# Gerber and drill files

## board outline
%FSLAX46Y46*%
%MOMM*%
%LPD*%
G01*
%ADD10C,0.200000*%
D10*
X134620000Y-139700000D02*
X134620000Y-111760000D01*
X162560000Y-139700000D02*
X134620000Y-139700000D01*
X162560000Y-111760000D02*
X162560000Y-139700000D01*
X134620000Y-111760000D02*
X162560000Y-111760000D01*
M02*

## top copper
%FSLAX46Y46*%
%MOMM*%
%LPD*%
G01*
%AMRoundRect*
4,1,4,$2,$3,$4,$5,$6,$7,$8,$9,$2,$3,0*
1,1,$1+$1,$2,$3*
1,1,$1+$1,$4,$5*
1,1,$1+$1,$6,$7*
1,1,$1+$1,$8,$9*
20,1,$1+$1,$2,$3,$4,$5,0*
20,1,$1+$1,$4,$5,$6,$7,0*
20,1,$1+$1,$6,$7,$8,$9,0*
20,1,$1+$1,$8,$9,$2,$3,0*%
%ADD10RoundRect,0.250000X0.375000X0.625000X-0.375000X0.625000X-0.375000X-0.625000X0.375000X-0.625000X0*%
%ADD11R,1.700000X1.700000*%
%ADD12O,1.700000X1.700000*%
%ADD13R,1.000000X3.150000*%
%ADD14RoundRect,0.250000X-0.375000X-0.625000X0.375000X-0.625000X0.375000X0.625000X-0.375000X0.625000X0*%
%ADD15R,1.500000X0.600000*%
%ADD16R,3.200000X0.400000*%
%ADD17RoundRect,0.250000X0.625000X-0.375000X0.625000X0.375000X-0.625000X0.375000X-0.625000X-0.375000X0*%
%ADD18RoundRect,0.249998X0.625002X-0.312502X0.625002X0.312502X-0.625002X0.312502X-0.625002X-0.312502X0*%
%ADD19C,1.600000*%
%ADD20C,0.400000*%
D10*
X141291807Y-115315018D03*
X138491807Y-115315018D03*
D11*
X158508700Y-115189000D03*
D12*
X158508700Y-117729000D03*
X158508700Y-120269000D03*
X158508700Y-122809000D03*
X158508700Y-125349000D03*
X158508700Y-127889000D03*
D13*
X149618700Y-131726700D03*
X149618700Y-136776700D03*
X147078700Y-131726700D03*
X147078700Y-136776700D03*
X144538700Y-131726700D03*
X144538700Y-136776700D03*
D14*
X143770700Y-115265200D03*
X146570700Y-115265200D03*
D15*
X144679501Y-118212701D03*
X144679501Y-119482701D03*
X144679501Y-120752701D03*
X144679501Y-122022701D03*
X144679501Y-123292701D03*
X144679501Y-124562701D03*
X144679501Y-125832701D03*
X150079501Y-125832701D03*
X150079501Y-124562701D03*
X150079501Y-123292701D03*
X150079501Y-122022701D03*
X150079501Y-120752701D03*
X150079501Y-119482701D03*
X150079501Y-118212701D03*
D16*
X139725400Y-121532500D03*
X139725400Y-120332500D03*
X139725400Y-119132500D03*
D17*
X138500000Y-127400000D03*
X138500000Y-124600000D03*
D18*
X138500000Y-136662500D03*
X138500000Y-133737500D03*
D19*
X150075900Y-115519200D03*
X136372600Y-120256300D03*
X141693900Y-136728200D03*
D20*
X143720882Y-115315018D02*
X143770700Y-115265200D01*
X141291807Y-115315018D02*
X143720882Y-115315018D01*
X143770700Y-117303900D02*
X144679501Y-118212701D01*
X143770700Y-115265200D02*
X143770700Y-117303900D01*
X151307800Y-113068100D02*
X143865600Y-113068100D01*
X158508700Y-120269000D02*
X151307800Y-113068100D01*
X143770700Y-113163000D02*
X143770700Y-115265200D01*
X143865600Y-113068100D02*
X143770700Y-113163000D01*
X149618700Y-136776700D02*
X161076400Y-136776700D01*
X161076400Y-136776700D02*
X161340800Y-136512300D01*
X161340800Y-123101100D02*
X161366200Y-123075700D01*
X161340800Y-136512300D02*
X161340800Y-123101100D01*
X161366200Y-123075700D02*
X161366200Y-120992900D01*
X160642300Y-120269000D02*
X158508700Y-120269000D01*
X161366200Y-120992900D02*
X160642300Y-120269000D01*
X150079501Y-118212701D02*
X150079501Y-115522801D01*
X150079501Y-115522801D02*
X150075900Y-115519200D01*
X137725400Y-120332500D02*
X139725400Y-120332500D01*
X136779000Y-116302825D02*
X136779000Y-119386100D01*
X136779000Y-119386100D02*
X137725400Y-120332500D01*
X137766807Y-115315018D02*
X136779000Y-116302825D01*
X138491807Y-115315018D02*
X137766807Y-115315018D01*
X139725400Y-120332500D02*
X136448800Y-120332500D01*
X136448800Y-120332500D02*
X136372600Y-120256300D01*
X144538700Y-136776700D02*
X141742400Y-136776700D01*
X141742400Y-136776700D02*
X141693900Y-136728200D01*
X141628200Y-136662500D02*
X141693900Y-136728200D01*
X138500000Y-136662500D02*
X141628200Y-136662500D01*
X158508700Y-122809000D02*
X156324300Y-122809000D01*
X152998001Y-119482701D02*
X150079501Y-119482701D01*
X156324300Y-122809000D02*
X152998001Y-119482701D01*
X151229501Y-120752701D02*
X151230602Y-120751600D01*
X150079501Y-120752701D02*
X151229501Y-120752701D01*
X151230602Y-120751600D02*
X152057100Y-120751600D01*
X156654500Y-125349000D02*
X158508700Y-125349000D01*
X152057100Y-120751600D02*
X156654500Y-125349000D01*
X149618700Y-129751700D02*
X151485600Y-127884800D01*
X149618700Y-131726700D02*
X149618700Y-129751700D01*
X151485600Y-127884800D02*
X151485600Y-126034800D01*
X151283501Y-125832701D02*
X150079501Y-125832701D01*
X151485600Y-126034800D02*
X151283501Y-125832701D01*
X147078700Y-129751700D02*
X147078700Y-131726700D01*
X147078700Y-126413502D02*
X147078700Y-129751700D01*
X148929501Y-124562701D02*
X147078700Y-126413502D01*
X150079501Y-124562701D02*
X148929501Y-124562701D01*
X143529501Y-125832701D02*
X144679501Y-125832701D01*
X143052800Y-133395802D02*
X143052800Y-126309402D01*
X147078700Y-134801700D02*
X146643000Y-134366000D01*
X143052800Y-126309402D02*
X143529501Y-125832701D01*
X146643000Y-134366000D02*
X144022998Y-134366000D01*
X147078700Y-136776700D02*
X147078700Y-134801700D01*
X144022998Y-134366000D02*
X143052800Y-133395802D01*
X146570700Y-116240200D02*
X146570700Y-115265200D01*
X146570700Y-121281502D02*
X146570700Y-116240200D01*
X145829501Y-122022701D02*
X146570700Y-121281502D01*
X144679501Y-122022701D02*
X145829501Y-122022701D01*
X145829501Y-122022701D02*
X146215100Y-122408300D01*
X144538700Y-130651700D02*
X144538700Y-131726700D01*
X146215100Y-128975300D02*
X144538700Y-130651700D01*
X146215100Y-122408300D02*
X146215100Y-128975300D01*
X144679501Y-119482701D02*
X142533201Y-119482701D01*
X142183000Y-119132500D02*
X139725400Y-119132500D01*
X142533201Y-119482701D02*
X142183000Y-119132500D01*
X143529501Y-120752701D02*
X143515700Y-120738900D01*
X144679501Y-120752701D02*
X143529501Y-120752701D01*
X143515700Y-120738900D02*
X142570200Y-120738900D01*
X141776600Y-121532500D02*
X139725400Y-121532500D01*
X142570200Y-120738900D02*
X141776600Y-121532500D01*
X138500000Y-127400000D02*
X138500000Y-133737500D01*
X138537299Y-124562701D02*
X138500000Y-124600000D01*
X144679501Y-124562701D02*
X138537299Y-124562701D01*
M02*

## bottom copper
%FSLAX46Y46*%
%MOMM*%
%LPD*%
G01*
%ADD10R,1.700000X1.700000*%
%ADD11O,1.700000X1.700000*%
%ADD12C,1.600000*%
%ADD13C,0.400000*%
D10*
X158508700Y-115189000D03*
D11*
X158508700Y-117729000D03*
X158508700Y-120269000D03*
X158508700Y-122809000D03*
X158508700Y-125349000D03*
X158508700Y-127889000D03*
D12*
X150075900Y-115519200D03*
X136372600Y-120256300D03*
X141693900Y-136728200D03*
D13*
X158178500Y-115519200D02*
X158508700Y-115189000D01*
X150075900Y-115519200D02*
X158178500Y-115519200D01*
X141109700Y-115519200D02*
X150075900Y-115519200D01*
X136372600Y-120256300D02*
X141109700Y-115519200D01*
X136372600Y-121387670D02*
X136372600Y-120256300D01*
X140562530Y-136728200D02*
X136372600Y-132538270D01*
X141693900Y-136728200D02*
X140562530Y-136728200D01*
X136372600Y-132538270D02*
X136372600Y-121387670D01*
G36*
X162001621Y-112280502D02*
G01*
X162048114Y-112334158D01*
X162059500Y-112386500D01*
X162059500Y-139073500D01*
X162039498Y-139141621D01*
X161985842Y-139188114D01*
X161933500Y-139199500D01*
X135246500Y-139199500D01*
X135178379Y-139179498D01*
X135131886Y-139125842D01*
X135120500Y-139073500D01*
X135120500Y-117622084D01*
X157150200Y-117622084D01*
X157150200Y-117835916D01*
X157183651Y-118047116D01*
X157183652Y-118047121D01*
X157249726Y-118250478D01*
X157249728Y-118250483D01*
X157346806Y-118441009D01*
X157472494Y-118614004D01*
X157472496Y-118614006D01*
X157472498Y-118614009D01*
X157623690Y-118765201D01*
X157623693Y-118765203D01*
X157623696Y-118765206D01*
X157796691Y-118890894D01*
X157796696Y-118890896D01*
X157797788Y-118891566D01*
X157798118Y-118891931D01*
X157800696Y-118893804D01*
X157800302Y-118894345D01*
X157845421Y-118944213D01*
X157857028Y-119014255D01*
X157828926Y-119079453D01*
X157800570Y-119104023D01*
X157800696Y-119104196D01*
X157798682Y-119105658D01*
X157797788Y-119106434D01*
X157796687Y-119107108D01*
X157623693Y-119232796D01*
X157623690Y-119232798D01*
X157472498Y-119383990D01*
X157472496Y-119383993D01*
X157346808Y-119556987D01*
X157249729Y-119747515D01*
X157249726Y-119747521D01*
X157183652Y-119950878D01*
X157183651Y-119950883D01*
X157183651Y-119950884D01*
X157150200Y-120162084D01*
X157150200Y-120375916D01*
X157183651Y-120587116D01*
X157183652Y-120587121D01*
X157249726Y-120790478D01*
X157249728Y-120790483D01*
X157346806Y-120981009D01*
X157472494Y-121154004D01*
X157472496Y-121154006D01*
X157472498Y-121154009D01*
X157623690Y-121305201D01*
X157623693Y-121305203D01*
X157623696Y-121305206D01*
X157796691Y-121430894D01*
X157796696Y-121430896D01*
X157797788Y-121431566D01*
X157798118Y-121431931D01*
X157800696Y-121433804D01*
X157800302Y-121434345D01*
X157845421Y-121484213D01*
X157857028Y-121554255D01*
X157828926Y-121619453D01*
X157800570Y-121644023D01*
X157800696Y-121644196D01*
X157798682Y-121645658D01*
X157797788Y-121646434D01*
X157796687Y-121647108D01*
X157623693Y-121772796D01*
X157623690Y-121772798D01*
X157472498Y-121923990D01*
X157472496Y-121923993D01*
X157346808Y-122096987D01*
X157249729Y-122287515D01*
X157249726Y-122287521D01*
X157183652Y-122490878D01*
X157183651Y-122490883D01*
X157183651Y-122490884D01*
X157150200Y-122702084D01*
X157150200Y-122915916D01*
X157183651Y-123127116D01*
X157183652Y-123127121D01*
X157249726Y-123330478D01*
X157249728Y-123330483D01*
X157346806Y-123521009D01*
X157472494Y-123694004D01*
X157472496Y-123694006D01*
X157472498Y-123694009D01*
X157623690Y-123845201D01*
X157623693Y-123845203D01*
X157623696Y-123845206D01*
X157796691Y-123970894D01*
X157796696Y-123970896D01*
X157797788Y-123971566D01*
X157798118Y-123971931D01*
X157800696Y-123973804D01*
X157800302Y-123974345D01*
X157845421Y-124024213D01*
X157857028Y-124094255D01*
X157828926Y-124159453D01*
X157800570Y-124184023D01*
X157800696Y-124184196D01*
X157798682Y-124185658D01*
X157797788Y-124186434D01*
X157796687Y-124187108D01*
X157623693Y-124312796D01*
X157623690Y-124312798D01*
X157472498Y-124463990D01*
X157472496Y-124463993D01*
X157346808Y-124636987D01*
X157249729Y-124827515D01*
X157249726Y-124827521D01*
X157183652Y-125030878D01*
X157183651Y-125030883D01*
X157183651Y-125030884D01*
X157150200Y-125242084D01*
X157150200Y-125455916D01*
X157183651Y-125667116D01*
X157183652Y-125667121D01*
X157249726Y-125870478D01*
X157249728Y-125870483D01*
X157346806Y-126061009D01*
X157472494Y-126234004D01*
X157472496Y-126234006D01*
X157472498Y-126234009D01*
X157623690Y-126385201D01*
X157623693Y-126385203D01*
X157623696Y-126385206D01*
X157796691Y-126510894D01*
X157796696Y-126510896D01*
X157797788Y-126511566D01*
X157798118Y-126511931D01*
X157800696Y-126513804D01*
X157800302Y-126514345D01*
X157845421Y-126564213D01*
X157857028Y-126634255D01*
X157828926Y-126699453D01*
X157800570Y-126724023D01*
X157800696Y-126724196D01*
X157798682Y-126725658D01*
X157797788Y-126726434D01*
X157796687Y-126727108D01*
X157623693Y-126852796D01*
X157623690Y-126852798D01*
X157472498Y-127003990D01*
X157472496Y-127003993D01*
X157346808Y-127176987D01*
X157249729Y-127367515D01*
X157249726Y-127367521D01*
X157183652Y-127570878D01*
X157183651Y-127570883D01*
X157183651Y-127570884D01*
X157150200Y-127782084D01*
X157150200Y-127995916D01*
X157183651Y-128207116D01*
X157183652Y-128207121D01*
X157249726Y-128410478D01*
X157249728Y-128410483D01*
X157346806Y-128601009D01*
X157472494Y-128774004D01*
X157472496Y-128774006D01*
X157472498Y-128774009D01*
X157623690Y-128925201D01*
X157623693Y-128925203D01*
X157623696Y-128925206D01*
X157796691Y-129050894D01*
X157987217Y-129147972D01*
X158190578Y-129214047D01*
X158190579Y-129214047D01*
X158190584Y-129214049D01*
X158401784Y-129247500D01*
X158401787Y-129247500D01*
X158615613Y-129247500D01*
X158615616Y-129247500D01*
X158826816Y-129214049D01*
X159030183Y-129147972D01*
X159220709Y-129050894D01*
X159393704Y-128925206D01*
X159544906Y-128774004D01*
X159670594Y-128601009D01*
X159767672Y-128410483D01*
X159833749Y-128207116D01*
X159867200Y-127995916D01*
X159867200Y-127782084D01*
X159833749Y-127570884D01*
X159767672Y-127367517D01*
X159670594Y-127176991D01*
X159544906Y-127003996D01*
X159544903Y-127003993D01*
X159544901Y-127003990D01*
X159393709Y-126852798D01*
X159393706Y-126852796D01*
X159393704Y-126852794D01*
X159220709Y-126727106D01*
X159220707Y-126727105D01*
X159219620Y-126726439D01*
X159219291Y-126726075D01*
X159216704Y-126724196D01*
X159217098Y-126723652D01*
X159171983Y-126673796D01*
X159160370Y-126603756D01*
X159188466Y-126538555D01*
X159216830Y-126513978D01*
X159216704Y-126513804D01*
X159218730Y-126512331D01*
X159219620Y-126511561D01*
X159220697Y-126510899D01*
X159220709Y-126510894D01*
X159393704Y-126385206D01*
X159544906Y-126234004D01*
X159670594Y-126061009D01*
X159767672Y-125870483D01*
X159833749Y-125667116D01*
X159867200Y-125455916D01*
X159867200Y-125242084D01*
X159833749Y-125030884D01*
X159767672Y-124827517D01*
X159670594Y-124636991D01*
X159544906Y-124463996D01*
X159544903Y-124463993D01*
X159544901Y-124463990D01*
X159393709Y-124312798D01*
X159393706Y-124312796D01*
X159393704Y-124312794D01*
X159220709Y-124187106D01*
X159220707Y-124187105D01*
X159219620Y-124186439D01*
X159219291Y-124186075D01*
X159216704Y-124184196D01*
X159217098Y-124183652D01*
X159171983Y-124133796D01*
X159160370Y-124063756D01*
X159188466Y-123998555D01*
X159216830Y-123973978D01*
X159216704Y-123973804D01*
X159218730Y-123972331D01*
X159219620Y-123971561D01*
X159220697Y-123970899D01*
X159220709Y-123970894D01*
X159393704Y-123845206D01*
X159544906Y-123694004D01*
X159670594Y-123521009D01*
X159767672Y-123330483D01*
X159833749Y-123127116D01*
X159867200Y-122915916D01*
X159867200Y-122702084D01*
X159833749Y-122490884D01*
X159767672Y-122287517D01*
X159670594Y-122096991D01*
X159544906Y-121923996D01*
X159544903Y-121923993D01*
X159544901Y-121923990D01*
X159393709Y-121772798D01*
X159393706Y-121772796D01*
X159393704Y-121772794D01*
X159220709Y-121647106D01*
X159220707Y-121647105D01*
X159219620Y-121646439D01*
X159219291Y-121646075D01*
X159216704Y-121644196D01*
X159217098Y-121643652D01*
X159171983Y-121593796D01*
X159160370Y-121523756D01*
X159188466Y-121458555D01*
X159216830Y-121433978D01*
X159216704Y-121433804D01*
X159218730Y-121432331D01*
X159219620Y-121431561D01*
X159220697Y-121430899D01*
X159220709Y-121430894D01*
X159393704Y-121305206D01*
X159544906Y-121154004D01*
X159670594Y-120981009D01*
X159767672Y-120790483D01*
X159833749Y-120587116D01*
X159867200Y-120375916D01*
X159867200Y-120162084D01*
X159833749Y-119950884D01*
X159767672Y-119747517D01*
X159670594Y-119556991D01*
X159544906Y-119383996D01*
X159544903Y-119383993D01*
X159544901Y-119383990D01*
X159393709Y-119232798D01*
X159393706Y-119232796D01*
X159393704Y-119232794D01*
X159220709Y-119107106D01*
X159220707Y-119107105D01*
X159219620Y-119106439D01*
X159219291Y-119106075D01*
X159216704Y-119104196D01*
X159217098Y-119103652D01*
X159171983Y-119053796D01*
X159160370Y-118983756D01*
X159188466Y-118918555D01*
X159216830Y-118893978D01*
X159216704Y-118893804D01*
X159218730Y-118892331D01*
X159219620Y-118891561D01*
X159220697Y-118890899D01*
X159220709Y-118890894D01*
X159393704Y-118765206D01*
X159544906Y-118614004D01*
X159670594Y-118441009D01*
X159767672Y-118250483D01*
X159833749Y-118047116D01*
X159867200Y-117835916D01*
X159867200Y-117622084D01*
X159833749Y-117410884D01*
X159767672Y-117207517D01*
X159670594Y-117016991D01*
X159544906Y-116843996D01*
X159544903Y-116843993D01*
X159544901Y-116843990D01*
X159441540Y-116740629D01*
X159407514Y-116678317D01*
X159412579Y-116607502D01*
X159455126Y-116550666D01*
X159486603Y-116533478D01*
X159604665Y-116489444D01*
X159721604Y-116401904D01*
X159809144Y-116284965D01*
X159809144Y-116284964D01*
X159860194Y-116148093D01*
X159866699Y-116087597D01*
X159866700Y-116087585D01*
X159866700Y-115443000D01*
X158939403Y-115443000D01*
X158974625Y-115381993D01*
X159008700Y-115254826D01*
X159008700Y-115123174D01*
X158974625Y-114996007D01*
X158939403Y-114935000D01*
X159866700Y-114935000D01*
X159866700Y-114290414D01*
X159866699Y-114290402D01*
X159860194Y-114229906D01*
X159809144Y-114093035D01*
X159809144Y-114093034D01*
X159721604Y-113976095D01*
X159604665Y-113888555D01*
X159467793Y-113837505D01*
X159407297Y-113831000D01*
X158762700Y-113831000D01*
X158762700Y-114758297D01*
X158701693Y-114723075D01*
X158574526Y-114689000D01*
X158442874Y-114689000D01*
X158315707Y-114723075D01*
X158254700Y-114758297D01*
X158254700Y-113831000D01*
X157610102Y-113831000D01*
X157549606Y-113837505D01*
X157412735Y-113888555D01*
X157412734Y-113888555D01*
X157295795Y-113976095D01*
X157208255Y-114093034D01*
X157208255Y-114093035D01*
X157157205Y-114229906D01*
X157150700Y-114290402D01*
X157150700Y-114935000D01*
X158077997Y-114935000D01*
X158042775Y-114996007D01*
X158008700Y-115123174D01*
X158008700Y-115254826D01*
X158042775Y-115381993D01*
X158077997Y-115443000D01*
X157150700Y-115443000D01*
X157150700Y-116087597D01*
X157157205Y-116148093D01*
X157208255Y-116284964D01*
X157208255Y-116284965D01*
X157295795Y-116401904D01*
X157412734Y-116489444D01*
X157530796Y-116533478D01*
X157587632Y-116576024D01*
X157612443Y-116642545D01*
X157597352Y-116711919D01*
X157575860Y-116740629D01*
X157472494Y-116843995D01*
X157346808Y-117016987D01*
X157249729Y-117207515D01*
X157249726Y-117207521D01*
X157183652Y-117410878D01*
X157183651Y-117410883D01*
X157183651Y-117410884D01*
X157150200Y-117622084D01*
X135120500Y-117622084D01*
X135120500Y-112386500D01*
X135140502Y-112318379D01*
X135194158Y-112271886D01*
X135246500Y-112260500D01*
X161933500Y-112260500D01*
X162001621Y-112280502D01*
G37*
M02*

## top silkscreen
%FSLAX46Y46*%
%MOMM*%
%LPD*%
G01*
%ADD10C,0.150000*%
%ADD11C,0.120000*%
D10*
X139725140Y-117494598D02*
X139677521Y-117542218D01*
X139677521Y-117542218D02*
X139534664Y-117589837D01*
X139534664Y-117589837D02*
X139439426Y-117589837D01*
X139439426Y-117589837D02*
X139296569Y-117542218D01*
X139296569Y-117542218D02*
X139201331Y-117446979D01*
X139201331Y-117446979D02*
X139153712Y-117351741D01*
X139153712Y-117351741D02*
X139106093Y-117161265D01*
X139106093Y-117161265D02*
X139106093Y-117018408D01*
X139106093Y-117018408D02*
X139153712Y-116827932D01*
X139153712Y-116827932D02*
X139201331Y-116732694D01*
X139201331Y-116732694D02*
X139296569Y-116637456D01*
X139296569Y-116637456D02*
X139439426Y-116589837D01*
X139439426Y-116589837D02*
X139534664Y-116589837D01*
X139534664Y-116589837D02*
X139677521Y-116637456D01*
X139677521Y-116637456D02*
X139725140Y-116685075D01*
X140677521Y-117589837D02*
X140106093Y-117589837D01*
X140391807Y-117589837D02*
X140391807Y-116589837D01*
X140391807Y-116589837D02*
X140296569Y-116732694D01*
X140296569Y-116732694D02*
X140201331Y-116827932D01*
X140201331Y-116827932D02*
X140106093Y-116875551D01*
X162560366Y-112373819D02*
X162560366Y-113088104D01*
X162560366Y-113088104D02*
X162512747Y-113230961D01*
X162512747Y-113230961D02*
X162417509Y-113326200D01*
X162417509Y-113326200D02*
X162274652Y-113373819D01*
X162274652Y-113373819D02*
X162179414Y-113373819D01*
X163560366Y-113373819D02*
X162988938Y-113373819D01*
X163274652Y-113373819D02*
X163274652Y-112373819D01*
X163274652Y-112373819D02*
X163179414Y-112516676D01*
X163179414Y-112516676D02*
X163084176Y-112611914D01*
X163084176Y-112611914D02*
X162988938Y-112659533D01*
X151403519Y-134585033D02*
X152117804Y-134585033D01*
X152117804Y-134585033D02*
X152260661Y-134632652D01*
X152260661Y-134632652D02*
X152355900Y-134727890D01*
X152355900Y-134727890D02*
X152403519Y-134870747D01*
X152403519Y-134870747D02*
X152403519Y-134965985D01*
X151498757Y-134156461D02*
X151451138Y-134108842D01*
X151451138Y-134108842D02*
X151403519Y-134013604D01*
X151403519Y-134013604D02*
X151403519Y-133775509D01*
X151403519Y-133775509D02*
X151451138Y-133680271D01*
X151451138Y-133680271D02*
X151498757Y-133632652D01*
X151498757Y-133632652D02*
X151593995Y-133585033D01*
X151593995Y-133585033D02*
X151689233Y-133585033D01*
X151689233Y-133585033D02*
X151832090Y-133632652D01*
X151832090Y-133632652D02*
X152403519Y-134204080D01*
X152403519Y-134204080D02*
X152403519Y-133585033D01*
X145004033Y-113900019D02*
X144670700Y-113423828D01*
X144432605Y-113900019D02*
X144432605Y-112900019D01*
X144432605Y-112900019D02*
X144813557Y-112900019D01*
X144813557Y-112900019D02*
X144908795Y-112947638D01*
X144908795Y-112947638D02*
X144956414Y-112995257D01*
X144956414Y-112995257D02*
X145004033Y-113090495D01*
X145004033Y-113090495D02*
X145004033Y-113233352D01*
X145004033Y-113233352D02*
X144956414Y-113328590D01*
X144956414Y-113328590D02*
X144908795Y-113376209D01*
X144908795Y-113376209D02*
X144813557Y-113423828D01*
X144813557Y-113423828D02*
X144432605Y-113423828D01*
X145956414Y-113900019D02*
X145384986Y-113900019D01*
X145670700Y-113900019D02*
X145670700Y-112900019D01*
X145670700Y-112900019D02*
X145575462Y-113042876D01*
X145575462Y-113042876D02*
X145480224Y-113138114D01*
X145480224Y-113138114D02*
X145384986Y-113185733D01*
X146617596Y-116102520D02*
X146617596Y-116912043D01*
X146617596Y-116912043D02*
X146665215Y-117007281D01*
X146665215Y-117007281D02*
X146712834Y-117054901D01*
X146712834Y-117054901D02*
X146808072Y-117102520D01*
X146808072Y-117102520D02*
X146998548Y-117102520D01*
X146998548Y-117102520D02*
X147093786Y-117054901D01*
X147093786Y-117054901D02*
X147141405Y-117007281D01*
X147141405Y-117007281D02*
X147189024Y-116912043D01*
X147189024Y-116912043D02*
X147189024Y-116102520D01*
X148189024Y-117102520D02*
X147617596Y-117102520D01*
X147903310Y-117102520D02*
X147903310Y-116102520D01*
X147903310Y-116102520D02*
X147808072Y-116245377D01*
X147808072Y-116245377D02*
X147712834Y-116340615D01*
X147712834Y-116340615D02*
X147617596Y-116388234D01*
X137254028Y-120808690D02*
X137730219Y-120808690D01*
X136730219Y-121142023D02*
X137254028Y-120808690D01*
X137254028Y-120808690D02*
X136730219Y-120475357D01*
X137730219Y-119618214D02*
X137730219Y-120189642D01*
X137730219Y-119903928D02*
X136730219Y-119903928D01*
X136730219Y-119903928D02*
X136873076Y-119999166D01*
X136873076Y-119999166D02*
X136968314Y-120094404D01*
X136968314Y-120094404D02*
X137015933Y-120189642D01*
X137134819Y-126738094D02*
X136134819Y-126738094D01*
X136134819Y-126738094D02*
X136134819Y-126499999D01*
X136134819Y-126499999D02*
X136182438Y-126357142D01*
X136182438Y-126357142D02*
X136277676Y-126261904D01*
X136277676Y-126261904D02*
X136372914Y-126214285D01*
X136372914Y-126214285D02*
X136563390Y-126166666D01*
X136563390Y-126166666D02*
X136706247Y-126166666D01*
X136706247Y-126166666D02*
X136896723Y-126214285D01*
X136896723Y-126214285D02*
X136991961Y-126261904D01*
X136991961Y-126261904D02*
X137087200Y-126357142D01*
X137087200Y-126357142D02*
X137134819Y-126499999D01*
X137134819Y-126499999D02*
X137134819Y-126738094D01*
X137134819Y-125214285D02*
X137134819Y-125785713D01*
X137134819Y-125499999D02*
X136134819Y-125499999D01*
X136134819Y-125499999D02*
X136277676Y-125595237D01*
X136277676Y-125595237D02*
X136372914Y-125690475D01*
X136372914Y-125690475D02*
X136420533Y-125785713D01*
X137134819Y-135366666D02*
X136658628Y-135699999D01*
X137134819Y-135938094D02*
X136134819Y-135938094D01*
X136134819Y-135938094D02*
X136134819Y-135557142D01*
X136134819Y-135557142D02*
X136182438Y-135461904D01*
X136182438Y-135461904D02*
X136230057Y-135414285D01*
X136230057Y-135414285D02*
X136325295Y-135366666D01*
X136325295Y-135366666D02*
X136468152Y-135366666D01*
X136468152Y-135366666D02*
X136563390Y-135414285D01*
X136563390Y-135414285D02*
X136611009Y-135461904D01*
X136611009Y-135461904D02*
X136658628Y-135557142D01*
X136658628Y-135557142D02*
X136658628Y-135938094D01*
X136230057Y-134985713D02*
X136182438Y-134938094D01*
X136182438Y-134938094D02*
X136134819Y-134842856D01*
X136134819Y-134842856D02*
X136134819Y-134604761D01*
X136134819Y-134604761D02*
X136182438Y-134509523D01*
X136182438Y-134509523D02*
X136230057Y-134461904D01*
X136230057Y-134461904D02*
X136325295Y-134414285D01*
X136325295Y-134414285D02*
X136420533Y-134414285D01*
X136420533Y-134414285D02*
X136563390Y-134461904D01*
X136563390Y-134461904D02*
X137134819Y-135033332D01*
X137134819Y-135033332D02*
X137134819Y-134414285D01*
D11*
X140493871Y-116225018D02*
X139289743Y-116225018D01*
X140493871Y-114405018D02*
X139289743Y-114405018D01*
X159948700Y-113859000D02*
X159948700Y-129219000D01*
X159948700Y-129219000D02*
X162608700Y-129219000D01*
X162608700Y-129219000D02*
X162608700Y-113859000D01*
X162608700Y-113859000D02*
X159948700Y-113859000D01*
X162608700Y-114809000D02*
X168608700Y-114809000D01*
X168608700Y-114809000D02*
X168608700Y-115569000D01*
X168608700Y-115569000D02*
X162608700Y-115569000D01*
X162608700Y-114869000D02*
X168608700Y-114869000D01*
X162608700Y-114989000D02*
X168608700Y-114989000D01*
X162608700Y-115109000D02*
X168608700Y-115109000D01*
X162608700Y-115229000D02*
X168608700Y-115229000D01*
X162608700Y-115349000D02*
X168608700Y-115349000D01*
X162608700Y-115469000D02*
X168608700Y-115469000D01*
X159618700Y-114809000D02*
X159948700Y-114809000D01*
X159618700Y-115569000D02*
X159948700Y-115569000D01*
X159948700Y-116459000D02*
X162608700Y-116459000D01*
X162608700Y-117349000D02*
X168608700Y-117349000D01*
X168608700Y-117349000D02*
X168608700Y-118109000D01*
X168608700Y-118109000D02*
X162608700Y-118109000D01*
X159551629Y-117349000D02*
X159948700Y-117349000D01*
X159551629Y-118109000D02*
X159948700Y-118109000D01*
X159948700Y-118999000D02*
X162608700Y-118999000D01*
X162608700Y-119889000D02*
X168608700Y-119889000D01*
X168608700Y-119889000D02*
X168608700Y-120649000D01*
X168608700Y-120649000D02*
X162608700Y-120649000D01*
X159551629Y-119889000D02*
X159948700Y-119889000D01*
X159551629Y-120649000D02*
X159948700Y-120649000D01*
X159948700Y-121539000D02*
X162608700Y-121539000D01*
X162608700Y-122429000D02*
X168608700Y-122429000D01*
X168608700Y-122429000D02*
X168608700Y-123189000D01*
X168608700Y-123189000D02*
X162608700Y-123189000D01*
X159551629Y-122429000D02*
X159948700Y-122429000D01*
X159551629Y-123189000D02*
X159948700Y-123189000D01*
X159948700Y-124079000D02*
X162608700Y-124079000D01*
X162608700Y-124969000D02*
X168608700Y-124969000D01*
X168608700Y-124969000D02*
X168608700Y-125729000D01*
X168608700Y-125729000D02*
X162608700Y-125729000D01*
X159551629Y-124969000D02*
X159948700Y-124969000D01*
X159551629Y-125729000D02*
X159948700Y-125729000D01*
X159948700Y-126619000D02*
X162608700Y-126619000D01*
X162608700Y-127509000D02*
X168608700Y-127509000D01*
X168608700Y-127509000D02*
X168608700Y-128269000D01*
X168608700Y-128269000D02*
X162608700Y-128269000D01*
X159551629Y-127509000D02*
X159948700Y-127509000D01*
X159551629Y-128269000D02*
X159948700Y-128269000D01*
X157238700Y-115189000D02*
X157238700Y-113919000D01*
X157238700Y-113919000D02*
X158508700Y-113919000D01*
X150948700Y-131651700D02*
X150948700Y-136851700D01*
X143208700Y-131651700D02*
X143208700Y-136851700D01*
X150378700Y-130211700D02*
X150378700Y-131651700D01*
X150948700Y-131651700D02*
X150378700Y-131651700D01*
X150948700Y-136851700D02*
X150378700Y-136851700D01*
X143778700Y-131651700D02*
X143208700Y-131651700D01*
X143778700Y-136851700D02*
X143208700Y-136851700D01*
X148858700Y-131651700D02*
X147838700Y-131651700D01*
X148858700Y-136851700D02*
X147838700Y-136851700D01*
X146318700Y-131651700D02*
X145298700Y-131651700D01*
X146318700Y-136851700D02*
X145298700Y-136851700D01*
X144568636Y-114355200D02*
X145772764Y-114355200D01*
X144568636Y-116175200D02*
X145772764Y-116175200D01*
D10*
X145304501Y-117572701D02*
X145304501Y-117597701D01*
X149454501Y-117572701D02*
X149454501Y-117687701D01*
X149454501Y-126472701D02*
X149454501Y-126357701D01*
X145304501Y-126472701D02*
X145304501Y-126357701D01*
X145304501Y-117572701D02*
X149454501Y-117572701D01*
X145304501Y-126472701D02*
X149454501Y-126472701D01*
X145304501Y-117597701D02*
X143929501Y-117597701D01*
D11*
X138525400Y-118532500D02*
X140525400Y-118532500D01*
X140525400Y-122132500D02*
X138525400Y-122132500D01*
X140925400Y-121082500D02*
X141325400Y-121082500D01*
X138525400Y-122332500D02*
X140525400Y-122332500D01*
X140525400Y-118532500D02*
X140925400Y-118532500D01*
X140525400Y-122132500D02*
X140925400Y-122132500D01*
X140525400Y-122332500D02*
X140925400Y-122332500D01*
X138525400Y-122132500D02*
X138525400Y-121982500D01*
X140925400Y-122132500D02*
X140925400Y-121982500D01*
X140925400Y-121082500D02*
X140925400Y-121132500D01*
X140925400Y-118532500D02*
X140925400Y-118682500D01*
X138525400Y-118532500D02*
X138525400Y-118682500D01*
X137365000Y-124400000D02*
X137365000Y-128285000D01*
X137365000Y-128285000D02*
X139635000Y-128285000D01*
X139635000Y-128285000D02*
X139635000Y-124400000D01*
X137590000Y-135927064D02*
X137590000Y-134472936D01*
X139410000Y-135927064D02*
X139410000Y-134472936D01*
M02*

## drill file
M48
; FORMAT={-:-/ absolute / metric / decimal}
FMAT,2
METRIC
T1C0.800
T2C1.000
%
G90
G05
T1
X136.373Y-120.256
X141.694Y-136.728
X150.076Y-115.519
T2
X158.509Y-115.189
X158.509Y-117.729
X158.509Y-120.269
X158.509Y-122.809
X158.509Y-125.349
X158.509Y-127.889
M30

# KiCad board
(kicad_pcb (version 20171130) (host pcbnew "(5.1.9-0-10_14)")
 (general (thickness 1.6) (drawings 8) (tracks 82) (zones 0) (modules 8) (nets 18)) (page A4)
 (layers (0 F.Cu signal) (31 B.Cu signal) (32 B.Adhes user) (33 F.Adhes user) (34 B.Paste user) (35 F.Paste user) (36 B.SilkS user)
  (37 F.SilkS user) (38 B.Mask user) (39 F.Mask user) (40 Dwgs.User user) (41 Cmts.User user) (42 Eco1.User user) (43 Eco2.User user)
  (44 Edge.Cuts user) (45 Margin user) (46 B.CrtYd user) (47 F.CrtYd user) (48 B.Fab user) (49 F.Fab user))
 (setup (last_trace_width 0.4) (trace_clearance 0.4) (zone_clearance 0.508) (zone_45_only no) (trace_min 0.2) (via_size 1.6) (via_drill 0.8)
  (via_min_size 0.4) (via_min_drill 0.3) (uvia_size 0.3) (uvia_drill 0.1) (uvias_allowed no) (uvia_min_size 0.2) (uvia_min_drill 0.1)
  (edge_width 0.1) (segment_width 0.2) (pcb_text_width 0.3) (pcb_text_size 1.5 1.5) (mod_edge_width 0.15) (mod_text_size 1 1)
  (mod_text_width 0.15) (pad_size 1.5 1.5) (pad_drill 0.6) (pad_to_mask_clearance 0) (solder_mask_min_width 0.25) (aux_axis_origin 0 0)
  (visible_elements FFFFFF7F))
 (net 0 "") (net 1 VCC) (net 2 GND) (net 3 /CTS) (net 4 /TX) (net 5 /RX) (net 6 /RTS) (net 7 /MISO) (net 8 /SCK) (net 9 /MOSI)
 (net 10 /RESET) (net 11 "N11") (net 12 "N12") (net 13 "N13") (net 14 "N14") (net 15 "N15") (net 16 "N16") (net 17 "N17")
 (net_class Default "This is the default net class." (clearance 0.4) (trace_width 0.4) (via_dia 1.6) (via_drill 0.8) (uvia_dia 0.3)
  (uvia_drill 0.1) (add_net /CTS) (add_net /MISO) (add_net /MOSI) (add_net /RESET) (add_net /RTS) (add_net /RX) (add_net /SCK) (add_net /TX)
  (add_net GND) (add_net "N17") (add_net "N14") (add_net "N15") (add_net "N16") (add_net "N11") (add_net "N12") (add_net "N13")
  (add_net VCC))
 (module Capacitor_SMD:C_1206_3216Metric (layer F.Cu) (at 139.891807 115.315018 180)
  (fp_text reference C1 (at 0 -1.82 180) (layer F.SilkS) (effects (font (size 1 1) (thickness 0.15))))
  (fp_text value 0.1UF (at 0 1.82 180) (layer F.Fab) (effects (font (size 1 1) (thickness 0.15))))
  (fp_line (start -0.602064 -0.91) (end 0.602064 -0.91) (layer F.SilkS) (width 0.12))
  (fp_line (start -0.602064 0.91) (end 0.602064 0.91) (layer F.SilkS) (width 0.12))
  (pad 1 smd roundrect (at -1.4 0 180) (size 1.25 1.75) (layers F.Cu F.Paste F.Mask) (roundrect_rratio 0.2) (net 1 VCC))
  (pad 2 smd roundrect (at 1.4 0 180) (size 1.25 1.75) (layers F.Cu F.Paste F.Mask) (roundrect_rratio 0.2) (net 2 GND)))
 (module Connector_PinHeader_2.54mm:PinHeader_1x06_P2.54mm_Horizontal (layer F.Cu) (at 158.5087 115.189)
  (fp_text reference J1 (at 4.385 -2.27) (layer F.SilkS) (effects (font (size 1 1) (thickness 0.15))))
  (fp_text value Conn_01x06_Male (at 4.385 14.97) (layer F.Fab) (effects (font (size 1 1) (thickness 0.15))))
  (fp_line (start 1.44 -1.33) (end 1.44 14.03) (layer F.SilkS) (width 0.12))
  (fp_line (start 1.44 14.03) (end 4.1 14.03) (layer F.SilkS) (width 0.12))
  (fp_line (start 4.1 14.03) (end 4.1 -1.33) (layer F.SilkS) (width 0.12))
  (fp_line (start 4.1 -1.33) (end 1.44 -1.33) (layer F.SilkS) (width 0.12))
  (fp_line (start 4.1 -0.38) (end 10.1 -0.38) (layer F.SilkS) (width 0.12))
  (fp_line (start 10.1 -0.38) (end 10.1 0.38) (layer F.SilkS) (width 0.12))
  (fp_line (start 10.1 0.38) (end 4.1 0.38) (layer F.SilkS) (width 0.12))
  (fp_line (start 4.1 -0.32) (end 10.1 -0.32) (layer F.SilkS) (width 0.12))
  (fp_line (start 4.1 -0.2) (end 10.1 -0.2) (layer F.SilkS) (width 0.12))
  (fp_line (start 4.1 -0.08) (end 10.1 -0.08) (layer F.SilkS) (width 0.12))
  (fp_line (start 4.1 0.04) (end 10.1 0.04) (layer F.SilkS) (width 0.12))
  (fp_line (start 4.1 0.16) (end 10.1 0.16) (layer F.SilkS) (width 0.12))
  (fp_line (start 4.1 0.28) (end 10.1 0.28) (layer F.SilkS) (width 0.12))
  (fp_line (start 1.11 -0.38) (end 1.44 -0.38) (layer F.SilkS) (width 0.12))
  (fp_line (start 1.11 0.38) (end 1.44 0.38) (layer F.SilkS) (width 0.12))
  (fp_line (start 1.44 1.27) (end 4.1 1.27) (layer F.SilkS) (width 0.12))
  (fp_line (start 4.1 2.16) (end 10.1 2.16) (layer F.SilkS) (width 0.12))
  (fp_line (start 10.1 2.16) (end 10.1 2.92) (layer F.SilkS) (width 0.12))
  (fp_line (start 10.1 2.92) (end 4.1 2.92) (layer F.SilkS) (width 0.12))
  (fp_line (start 1.042929 2.16) (end 1.44 2.16) (layer F.SilkS) (width 0.12))
  (fp_line (start 1.042929 2.92) (end 1.44 2.92) (layer F.SilkS) (width 0.12))
  (fp_line (start 1.44 3.81) (end 4.1 3.81) (layer F.SilkS) (width 0.12))
  (fp_line (start 4.1 4.7) (end 10.1 4.7) (layer F.SilkS) (width 0.12))
  (fp_line (start 10.1 4.7) (end 10.1 5.46) (layer F.SilkS) (width 0.12))
  (fp_line (start 10.1 5.46) (end 4.1 5.46) (layer F.SilkS) (width 0.12))
  (fp_line (start 1.042929 4.7) (end 1.44 4.7) (layer F.SilkS) (width 0.12))
  (fp_line (start 1.042929 5.46) (end 1.44 5.46) (layer F.SilkS) (width 0.12))
  (fp_line (start 1.44 6.35) (end 4.1 6.35) (layer F.SilkS) (width 0.12))
  (fp_line (start 4.1 7.24) (end 10.1 7.24) (layer F.SilkS) (width 0.12))
  (fp_line (start 10.1 7.24) (end 10.1 8) (layer F.SilkS) (width 0.12))
  (fp_line (start 10.1 8) (end 4.1 8) (layer F.SilkS) (width 0.12))
  (fp_line (start 1.042929 7.24) (end 1.44 7.24) (layer F.SilkS) (width 0.12))
  (fp_line (start 1.042929 8) (end 1.44 8) (layer F.SilkS) (width 0.12))
  (fp_line (start 1.44 8.89) (end 4.1 8.89) (layer F.SilkS) (width 0.12))
  (fp_line (start 4.1 9.78) (end 10.1 9.78) (layer F.SilkS) (width 0.12))
  (fp_line (start 10.1 9.78) (end 10.1 10.54) (layer F.SilkS) (width 0.12))
  (fp_line (start 10.1 10.54) (end 4.1 10.54) (layer F.SilkS) (width 0.12))
  (fp_line (start 1.042929 9.78) (end 1.44 9.78) (layer F.SilkS) (width 0.12))
  (fp_line (start 1.042929 10.54) (end 1.44 10.54) (layer F.SilkS) (width 0.12))
  (fp_line (start 1.44 11.43) (end 4.1 11.43) (layer F.SilkS) (width 0.12))
  (fp_line (start 4.1 12.32) (end 10.1 12.32) (layer F.SilkS) (width 0.12))
  (fp_line (start 10.1 12.32) (end 10.1 13.08) (layer F.SilkS) (width 0.12))
  (fp_line (start 10.1 13.08) (end 4.1 13.08) (layer F.SilkS) (width 0.12))
  (fp_line (start 1.042929 12.32) (end 1.44 12.32) (layer F.SilkS) (width 0.12))
  (fp_line (start 1.042929 13.08) (end 1.44 13.08) (layer F.SilkS) (width 0.12))
  (fp_line (start -1.27 0) (end -1.27 -1.27) (layer F.SilkS) (width 0.12))
  (fp_line (start -1.27 -1.27) (end 0 -1.27) (layer F.SilkS) (width 0.12))
  (pad 1 thru_hole rect (at 0 0) (size 1.7 1.7) (drill 1) (layers *.Cu *.Mask) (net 2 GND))
  (pad 2 thru_hole oval (at 0 2.54) (size 1.7 1.7) (drill 1) (layers *.Cu *.Mask) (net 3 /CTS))
  (pad 3 thru_hole oval (at 0 5.08) (size 1.7 1.7) (drill 1) (layers *.Cu *.Mask) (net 1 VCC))
  (pad 4 thru_hole oval (at 0 7.62) (size 1.7 1.7) (drill 1) (layers *.Cu *.Mask) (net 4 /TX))
  (pad 5 thru_hole oval (at 0 10.16) (size 1.7 1.7) (drill 1) (layers *.Cu *.Mask) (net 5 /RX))
  (pad 6 thru_hole oval (at 0 12.7) (size 1.7 1.7) (drill 1) (layers *.Cu *.Mask) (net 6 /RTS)))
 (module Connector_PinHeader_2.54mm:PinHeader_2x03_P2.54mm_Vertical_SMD (layer F.Cu) (at 147.0787 134.2517 270)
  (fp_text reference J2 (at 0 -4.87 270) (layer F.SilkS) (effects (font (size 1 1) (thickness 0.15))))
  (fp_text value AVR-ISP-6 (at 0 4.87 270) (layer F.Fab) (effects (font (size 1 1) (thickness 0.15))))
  (fp_line (start -2.6 -3.87) (end 2.6 -3.87) (layer F.SilkS) (width 0.12))
  (fp_line (start -2.6 3.87) (end 2.6 3.87) (layer F.SilkS) (width 0.12))
  (fp_line (start -4.04 -3.3) (end -2.6 -3.3) (layer F.SilkS) (width 0.12))
  (fp_line (start -2.6 -3.87) (end -2.6 -3.3) (layer F.SilkS) (width 0.12))
  (fp_line (start 2.6 -3.87) (end 2.6 -3.3) (layer F.SilkS) (width 0.12))
  (fp_line (start -2.6 3.3) (end -2.6 3.87) (layer F.SilkS) (width 0.12))
  (fp_line (start 2.6 3.3) (end 2.6 3.87) (layer F.SilkS) (width 0.12))
  (fp_line (start -2.6 -1.78) (end -2.6 -0.76) (layer F.SilkS) (width 0.12))
  (fp_line (start 2.6 -1.78) (end 2.6 -0.76) (layer F.SilkS) (width 0.12))
  (fp_line (start -2.6 0.76) (end -2.6 1.78) (layer F.SilkS) (width 0.12))
  (fp_line (start 2.6 0.76) (end 2.6 1.78) (layer F.SilkS) (width 0.12))
  (pad 1 smd rect (at -2.525 -2.54 270) (size 3.15 1) (layers F.Cu F.Paste F.Mask) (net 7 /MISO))
  (pad 2 smd rect (at 2.525 -2.54 270) (size 3.15 1) (layers F.Cu F.Paste F.Mask) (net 1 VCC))
  (pad 3 smd rect (at -2.525 0 270) (size 3.15 1) (layers F.Cu F.Paste F.Mask) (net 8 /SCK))
  (pad 4 smd rect (at 2.525 0 270) (size 3.15 1) (layers F.Cu F.Paste F.Mask) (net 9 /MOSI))
  (pad 5 smd rect (at -2.525 2.54 270) (size 3.15 1) (layers F.Cu F.Paste F.Mask) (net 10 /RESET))
  (pad 6 smd rect (at 2.525 2.54 270) (size 3.15 1) (layers F.Cu F.Paste F.Mask) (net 2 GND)))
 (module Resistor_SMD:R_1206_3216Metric (layer F.Cu) (at 145.1707 115.2652)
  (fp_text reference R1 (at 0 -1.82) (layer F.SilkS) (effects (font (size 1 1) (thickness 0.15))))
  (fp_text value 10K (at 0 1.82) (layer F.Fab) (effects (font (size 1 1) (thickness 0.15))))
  (fp_line (start -0.602064 -0.91) (end 0.602064 -0.91) (layer F.SilkS) (width 0.12))
  (fp_line (start -0.602064 0.91) (end 0.602064 0.91) (layer F.SilkS) (width 0.12))
  (pad 1 smd roundrect (at -1.4 0) (size 1.25 1.75) (layers F.Cu F.Paste F.Mask) (roundrect_rratio 0.2) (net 1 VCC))
  (pad 2 smd roundrect (at 1.4 0) (size 1.25 1.75) (layers F.Cu F.Paste F.Mask) (roundrect_rratio 0.2) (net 10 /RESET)))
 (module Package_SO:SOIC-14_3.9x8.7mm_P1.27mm (layer F.Cu) (at 147.379501 122.022701)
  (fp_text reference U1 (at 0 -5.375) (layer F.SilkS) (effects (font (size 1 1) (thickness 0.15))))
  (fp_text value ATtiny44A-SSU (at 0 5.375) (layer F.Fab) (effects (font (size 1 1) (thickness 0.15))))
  (fp_line (start -2.075 -4.45) (end -2.075 -4.425) (layer F.SilkS) (width 0.15))
  (fp_line (start 2.075 -4.45) (end 2.075 -4.335) (layer F.SilkS) (width 0.15))
  (fp_line (start 2.075 4.45) (end 2.075 4.335) (layer F.SilkS) (width 0.15))
  (fp_line (start -2.075 4.45) (end -2.075 4.335) (layer F.SilkS) (width 0.15))
  (fp_line (start -2.075 -4.45) (end 2.075 -4.45) (layer F.SilkS) (width 0.15))
  (fp_line (start -2.075 4.45) (end 2.075 4.45) (layer F.SilkS) (width 0.15))
  (fp_line (start -2.075 -4.425) (end -3.45 -4.425) (layer F.SilkS) (width 0.15))
  (pad 1 smd rect (at -2.7 -3.81) (size 1.5 0.6) (layers F.Cu F.Paste F.Mask) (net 1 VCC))
  (pad 2 smd rect (at -2.7 -2.54) (size 1.5 0.6) (layers F.Cu F.Paste F.Mask) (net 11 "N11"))
  (pad 3 smd rect (at -2.7 -1.27) (size 1.5 0.6) (layers F.Cu F.Paste F.Mask) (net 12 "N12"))
  (pad 4 smd rect (at -2.7 0) (size 1.5 0.6) (layers F.Cu F.Paste F.Mask) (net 10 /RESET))
  (pad 5 smd rect (at -2.7 1.27) (size 1.5 0.6) (layers F.Cu F.Paste F.Mask) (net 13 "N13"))
  (pad 6 smd rect (at -2.7 2.54) (size 1.5 0.6) (layers F.Cu F.Paste F.Mask) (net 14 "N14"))
  (pad 7 smd rect (at -2.7 3.81) (size 1.5 0.6) (layers F.Cu F.Paste F.Mask) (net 9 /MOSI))
  (pad 8 smd rect (at 2.7 3.81) (size 1.5 0.6) (layers F.Cu F.Paste F.Mask) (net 7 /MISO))
  (pad 9 smd rect (at 2.7 2.54) (size 1.5 0.6) (layers F.Cu F.Paste F.Mask) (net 8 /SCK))
  (pad 10 smd rect (at 2.7 1.27) (size 1.5 0.6) (layers F.Cu F.Paste F.Mask) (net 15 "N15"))
  (pad 11 smd rect (at 2.7 0) (size 1.5 0.6) (layers F.Cu F.Paste F.Mask) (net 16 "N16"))
  (pad 12 smd rect (at 2.7 -1.27) (size 1.5 0.6) (layers F.Cu F.Paste F.Mask) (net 5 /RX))
  (pad 13 smd rect (at 2.7 -2.54) (size 1.5 0.6) (layers F.Cu F.Paste F.Mask) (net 4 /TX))
  (pad 14 smd rect (at 2.7 -3.81) (size 1.5 0.6) (layers F.Cu F.Paste F.Mask) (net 2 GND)))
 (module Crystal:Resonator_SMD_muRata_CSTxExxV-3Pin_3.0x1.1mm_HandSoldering (layer F.Cu) (at 139.7254 120.3325 90)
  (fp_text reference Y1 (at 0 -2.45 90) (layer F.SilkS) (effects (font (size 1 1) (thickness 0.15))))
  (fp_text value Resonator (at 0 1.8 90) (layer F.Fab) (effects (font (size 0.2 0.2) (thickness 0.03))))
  (fp_line (start 1.8 -1.2) (end 1.8 0.8) (layer F.SilkS) (width 0.12))
  (fp_line (start -1.8 0.8) (end -1.8 -1.2) (layer F.SilkS) (width 0.12))
  (fp_line (start -0.75 1.2) (end -0.75 1.6) (layer F.SilkS) (width 0.12))
  (fp_line (start -2 -1.2) (end -2 0.8) (layer F.SilkS) (width 0.12))
  (fp_line (start 1.8 0.8) (end 1.8 1.2) (layer F.SilkS) (width 0.12))
  (fp_line (start -1.8 0.8) (end -1.8 1.2) (layer F.SilkS) (width 0.12))
  (fp_line (start -2 0.8) (end -2 1.2) (layer F.SilkS) (width 0.12))
  (fp_line (start -1.8 -1.2) (end -1.65 -1.2) (layer F.SilkS) (width 0.12))
  (fp_line (start -1.8 1.2) (end -1.65 1.2) (layer F.SilkS) (width 0.12))
  (fp_line (start -0.75 1.2) (end -0.8 1.2) (layer F.SilkS) (width 0.12))
  (fp_line (start 1.8 1.2) (end 1.65 1.2) (layer F.SilkS) (width 0.12))
  (fp_line (start 1.8 -1.2) (end 1.65 -1.2) (layer F.SilkS) (width 0.12))
  (pad 1 smd rect (at -1.2 0 90) (size 0.4 3.2) (layers F.Cu F.Paste F.Mask) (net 12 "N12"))
  (pad 2 smd rect (at 0 0 90) (size 0.4 3.2) (layers F.Cu F.Paste F.Mask) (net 2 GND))
  (pad 3 smd rect (at 1.2 0 90) (size 0.4 3.2) (layers F.Cu F.Paste F.Mask) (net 11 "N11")))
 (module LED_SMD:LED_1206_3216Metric (layer F.Cu) (at 138.5 126 90)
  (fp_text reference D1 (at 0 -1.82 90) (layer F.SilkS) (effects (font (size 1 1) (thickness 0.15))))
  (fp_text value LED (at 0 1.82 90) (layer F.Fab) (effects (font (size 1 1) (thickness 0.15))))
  (fp_line (start 1.6 -1.135) (end -2.285 -1.135) (layer F.SilkS) (width 0.12))
  (fp_line (start -2.285 -1.135) (end -2.285 1.135) (layer F.SilkS) (width 0.12))
  (fp_line (start -2.285 1.135) (end 1.6 1.135) (layer F.SilkS) (width 0.12))
  (pad 1 smd roundrect (at -1.4 0 90) (size 1.25 1.75) (layers F.Cu F.Paste F.Mask) (roundrect_rratio 0.2) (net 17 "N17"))
  (pad 2 smd roundrect (at 1.4 0 90) (size 1.25 1.75) (layers F.Cu F.Paste F.Mask) (roundrect_rratio 0.2) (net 14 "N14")))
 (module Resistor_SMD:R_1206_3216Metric (layer F.Cu) (at 138.5 135.2 90)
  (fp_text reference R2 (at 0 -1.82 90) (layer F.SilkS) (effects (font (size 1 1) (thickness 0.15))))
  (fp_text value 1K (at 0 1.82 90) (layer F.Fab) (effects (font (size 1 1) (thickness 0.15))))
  (fp_line (start -0.727064 -0.91) (end 0.727064 -0.91) (layer F.SilkS) (width 0.12))
  (fp_line (start -0.727064 0.91) (end 0.727064 0.91) (layer F.SilkS) (width 0.12))
  (pad 1 smd roundrect (at -1.4625 0 90) (size 1.125 1.75) (layers F.Cu F.Paste F.Mask) (roundrect_rratio 0.2222204444444444) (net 2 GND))
  (pad 2 smd roundrect (at 1.4625 0 90) (size 1.125 1.75) (layers F.Cu F.Paste F.Mask) (roundrect_rratio 0.2222204444444444) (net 17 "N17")))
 (gr_line (start 134.62 139.7) (end 134.62 111.76) (layer Edge.Cuts) (width 0.2))
 (gr_line (start 162.56 139.7) (end 134.62 139.7) (layer Edge.Cuts) (width 0.2))
 (gr_line (start 162.56 111.76) (end 162.56 139.7) (layer Edge.Cuts) (width 0.2))
 (gr_line (start 134.62 111.76) (end 162.56 111.76) (layer Edge.Cuts) (width 0.2))
 (segment (start 143.720882 115.315018) (end 143.7707 115.2652) (width 0.4) (layer F.Cu) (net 1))
 (segment (start 141.291807 115.315018) (end 143.720882 115.315018) (width 0.4) (layer F.Cu) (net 1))
 (segment (start 143.7707 117.3039) (end 144.679501 118.212701) (width 0.4) (layer F.Cu) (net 1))
 (segment (start 143.7707 115.2652) (end 143.7707 117.3039) (width 0.4) (layer F.Cu) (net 1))
 (segment (start 151.3078 113.0681) (end 143.8656 113.0681) (width 0.4) (layer F.Cu) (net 1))
 (segment (start 158.5087 120.269) (end 151.3078 113.0681) (width 0.4) (layer F.Cu) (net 1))
 (segment (start 143.7707 113.163) (end 143.7707 115.2652) (width 0.4) (layer F.Cu) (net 1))
 (segment (start 143.8656 113.0681) (end 143.7707 113.163) (width 0.4) (layer F.Cu) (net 1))
 (segment (start 149.6187 136.7767) (end 161.0764 136.7767) (width 0.4) (layer F.Cu) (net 1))
 (segment (start 161.0764 136.7767) (end 161.3408 136.5123) (width 0.4) (layer F.Cu) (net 1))
 (segment (start 161.3408 123.1011) (end 161.3662 123.0757) (width 0.4) (layer F.Cu) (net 1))
 (segment (start 161.3408 136.5123) (end 161.3408 123.1011) (width 0.4) (layer F.Cu) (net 1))
 (segment (start 161.3662 123.0757) (end 161.3662 120.9929) (width 0.4) (layer F.Cu) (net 1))
 (segment (start 160.6423 120.269) (end 158.5087 120.269) (width 0.4) (layer F.Cu) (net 1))
 (segment (start 161.3662 120.9929) (end 160.6423 120.269) (width 0.4) (layer F.Cu) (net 1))
 (via (at 150.0759 115.5192) (size 1.6) (drill 0.8) (layers F.Cu B.Cu) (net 2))
 (segment (start 150.079501 118.212701) (end 150.079501 115.522801) (width 0.4) (layer F.Cu) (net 2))
 (segment (start 150.079501 115.522801) (end 150.0759 115.5192) (width 0.4) (layer F.Cu) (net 2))
 (segment (start 158.1785 115.5192) (end 158.5087 115.189) (width 0.4) (layer B.Cu) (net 2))
 (segment (start 150.0759 115.5192) (end 158.1785 115.5192) (width 0.4) (layer B.Cu) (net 2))
 (segment (start 137.7254 120.3325) (end 139.7254 120.3325) (width 0.4) (layer F.Cu) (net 2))
 (segment (start 136.779 116.302825) (end 136.779 119.3861) (width 0.4) (layer F.Cu) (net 2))
 (segment (start 136.779 119.3861) (end 137.7254 120.3325) (width 0.4) (layer F.Cu) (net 2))
 (segment (start 137.766807 115.315018) (end 136.779 116.302825) (width 0.4) (layer F.Cu) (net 2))
 (segment (start 138.491807 115.315018) (end 137.766807 115.315018) (width 0.4) (layer F.Cu) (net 2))
 (via (at 136.3726 120.2563) (size 1.6) (drill 0.8) (layers F.Cu B.Cu) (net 2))
 (segment (start 139.7254 120.3325) (end 136.4488 120.3325) (width 0.4) (layer F.Cu) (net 2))
 (segment (start 136.4488 120.3325) (end 136.3726 120.2563) (width 0.4) (layer F.Cu) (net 2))
 (segment (start 141.1097 115.5192) (end 150.0759 115.5192) (width 0.4) (layer B.Cu) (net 2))
 (segment (start 136.3726 120.2563) (end 141.1097 115.5192) (width 0.4) (layer B.Cu) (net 2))
 (via (at 141.6939 136.7282) (size 1.6) (drill 0.8) (layers F.Cu B.Cu) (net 2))
 (segment (start 144.5387 136.7767) (end 141.7424 136.7767) (width 0.4) (layer F.Cu) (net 2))
 (segment (start 141.7424 136.7767) (end 141.6939 136.7282) (width 0.4) (layer F.Cu) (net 2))
 (segment (start 136.3726 121.38767) (end 136.3726 120.2563) (width 0.4) (layer B.Cu) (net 2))
 (segment (start 140.56253 136.7282) (end 136.3726 132.53827) (width 0.4) (layer B.Cu) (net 2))
 (segment (start 141.6939 136.7282) (end 140.56253 136.7282) (width 0.4) (layer B.Cu) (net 2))
 (segment (start 136.3726 132.53827) (end 136.3726 121.38767) (width 0.4) (layer B.Cu) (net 2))
 (segment (start 141.6282 136.6625) (end 141.6939 136.7282) (width 0.4) (layer F.Cu) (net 2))
 (segment (start 138.5 136.6625) (end 141.6282 136.6625) (width 0.4) (layer F.Cu) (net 2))
 (segment (start 158.5087 122.809) (end 156.3243 122.809) (width 0.4) (layer F.Cu) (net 4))
 (segment (start 152.998001 119.482701) (end 150.079501 119.482701) (width 0.4) (layer F.Cu) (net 4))
 (segment (start 156.3243 122.809) (end 152.998001 119.482701) (width 0.4) (layer F.Cu) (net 4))
 (segment (start 151.229501 120.752701) (end 151.230602 120.7516) (width 0.4) (layer F.Cu) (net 5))
 (segment (start 150.079501 120.752701) (end 151.229501 120.752701) (width 0.4) (layer F.Cu) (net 5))
 (segment (start 151.230602 120.7516) (end 152.0571 120.7516) (width 0.4) (layer F.Cu) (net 5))
 (segment (start 156.6545 125.349) (end 158.5087 125.349) (width 0.4) (layer F.Cu) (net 5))
 (segment (start 152.0571 120.7516) (end 156.6545 125.349) (width 0.4) (layer F.Cu) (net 5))
 (segment (start 149.6187 129.7517) (end 151.4856 127.8848) (width 0.4) (layer F.Cu) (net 7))
 (segment (start 149.6187 131.7267) (end 149.6187 129.7517) (width 0.4) (layer F.Cu) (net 7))
 (segment (start 151.4856 127.8848) (end 151.4856 126.0348) (width 0.4) (layer F.Cu) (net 7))
 (segment (start 151.283501 125.832701) (end 150.079501 125.832701) (width 0.4) (layer F.Cu) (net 7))
 (segment (start 151.4856 126.0348) (end 151.283501 125.832701) (width 0.4) (layer F.Cu) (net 7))
 (segment (start 147.0787 129.7517) (end 147.0787 131.7267) (width 0.4) (layer F.Cu) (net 8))
 (segment (start 147.0787 126.413502) (end 147.0787 129.7517) (width 0.4) (layer F.Cu) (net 8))
 (segment (start 148.929501 124.562701) (end 147.0787 126.413502) (width 0.4) (layer F.Cu) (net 8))
 (segment (start 150.079501 124.562701) (end 148.929501 124.562701) (width 0.4) (layer F.Cu) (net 8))
 (segment (start 143.529501 125.832701) (end 144.679501 125.832701) (width 0.4) (layer F.Cu) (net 9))
 (segment (start 143.0528 133.395802) (end 143.0528 126.309402) (width 0.4) (layer F.Cu) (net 9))
 (segment (start 147.0787 134.8017) (end 146.643 134.366) (width 0.4) (layer F.Cu) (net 9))
 (segment (start 143.0528 126.309402) (end 143.529501 125.832701) (width 0.4) (layer F.Cu) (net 9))
 (segment (start 146.643 134.366) (end 144.022998 134.366) (width 0.4) (layer F.Cu) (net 9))
 (segment (start 147.0787 136.7767) (end 147.0787 134.8017) (width 0.4) (layer F.Cu) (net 9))
 (segment (start 144.022998 134.366) (end 143.0528 133.395802) (width 0.4) (layer F.Cu) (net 9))
 (segment (start 146.5707 116.2402) (end 146.5707 115.2652) (width 0.4) (layer F.Cu) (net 10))
 (segment (start 146.5707 121.281502) (end 146.5707 116.2402) (width 0.4) (layer F.Cu) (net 10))
 (segment (start 145.829501 122.022701) (end 146.5707 121.281502) (width 0.4) (layer F.Cu) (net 10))
 (segment (start 144.679501 122.022701) (end 145.829501 122.022701) (width 0.4) (layer F.Cu) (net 10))
 (segment (start 145.829501 122.022701) (end 146.2151 122.4083) (width 0.4) (layer F.Cu) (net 10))
 (segment (start 144.5387 130.6517) (end 144.5387 131.7267) (width 0.4) (layer F.Cu) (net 10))
 (segment (start 146.2151 128.9753) (end 144.5387 130.6517) (width 0.4) (layer F.Cu) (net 10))
 (segment (start 146.2151 122.4083) (end 146.2151 128.9753) (width 0.4) (layer F.Cu) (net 10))
 (segment (start 144.679501 119.482701) (end 142.533201 119.482701) (width 0.4) (layer F.Cu) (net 11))
 (segment (start 142.183 119.1325) (end 139.7254 119.1325) (width 0.4) (layer F.Cu) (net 11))
 (segment (start 142.533201 119.482701) (end 142.183 119.1325) (width 0.4) (layer F.Cu) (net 11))
 (segment (start 143.529501 120.752701) (end 143.5157 120.7389) (width 0.4) (layer F.Cu) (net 12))
 (segment (start 144.679501 120.752701) (end 143.529501 120.752701) (width 0.4) (layer F.Cu) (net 12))
 (segment (start 143.5157 120.7389) (end 142.5702 120.7389) (width 0.4) (layer F.Cu) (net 12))
 (segment (start 141.7766 121.5325) (end 139.7254 121.5325) (width 0.4) (layer F.Cu) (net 12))
 (segment (start 142.5702 120.7389) (end 141.7766 121.5325) (width 0.4) (layer F.Cu) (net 12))
 (segment (start 138.5 127.4) (end 138.5 133.7375) (width 0.4) (layer F.Cu) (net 17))
 (segment (start 138.537299 124.562701) (end 138.5 124.6) (width 0.4) (layer F.Cu) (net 14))
 (segment (start 144.679501 124.562701) (end 138.537299 124.562701) (width 0.4) (layer F.Cu) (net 14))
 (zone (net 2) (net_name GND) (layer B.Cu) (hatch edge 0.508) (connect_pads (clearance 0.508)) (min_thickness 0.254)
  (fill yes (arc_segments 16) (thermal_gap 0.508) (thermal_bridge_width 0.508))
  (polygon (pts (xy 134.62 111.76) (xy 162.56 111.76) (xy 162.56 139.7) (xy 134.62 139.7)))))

